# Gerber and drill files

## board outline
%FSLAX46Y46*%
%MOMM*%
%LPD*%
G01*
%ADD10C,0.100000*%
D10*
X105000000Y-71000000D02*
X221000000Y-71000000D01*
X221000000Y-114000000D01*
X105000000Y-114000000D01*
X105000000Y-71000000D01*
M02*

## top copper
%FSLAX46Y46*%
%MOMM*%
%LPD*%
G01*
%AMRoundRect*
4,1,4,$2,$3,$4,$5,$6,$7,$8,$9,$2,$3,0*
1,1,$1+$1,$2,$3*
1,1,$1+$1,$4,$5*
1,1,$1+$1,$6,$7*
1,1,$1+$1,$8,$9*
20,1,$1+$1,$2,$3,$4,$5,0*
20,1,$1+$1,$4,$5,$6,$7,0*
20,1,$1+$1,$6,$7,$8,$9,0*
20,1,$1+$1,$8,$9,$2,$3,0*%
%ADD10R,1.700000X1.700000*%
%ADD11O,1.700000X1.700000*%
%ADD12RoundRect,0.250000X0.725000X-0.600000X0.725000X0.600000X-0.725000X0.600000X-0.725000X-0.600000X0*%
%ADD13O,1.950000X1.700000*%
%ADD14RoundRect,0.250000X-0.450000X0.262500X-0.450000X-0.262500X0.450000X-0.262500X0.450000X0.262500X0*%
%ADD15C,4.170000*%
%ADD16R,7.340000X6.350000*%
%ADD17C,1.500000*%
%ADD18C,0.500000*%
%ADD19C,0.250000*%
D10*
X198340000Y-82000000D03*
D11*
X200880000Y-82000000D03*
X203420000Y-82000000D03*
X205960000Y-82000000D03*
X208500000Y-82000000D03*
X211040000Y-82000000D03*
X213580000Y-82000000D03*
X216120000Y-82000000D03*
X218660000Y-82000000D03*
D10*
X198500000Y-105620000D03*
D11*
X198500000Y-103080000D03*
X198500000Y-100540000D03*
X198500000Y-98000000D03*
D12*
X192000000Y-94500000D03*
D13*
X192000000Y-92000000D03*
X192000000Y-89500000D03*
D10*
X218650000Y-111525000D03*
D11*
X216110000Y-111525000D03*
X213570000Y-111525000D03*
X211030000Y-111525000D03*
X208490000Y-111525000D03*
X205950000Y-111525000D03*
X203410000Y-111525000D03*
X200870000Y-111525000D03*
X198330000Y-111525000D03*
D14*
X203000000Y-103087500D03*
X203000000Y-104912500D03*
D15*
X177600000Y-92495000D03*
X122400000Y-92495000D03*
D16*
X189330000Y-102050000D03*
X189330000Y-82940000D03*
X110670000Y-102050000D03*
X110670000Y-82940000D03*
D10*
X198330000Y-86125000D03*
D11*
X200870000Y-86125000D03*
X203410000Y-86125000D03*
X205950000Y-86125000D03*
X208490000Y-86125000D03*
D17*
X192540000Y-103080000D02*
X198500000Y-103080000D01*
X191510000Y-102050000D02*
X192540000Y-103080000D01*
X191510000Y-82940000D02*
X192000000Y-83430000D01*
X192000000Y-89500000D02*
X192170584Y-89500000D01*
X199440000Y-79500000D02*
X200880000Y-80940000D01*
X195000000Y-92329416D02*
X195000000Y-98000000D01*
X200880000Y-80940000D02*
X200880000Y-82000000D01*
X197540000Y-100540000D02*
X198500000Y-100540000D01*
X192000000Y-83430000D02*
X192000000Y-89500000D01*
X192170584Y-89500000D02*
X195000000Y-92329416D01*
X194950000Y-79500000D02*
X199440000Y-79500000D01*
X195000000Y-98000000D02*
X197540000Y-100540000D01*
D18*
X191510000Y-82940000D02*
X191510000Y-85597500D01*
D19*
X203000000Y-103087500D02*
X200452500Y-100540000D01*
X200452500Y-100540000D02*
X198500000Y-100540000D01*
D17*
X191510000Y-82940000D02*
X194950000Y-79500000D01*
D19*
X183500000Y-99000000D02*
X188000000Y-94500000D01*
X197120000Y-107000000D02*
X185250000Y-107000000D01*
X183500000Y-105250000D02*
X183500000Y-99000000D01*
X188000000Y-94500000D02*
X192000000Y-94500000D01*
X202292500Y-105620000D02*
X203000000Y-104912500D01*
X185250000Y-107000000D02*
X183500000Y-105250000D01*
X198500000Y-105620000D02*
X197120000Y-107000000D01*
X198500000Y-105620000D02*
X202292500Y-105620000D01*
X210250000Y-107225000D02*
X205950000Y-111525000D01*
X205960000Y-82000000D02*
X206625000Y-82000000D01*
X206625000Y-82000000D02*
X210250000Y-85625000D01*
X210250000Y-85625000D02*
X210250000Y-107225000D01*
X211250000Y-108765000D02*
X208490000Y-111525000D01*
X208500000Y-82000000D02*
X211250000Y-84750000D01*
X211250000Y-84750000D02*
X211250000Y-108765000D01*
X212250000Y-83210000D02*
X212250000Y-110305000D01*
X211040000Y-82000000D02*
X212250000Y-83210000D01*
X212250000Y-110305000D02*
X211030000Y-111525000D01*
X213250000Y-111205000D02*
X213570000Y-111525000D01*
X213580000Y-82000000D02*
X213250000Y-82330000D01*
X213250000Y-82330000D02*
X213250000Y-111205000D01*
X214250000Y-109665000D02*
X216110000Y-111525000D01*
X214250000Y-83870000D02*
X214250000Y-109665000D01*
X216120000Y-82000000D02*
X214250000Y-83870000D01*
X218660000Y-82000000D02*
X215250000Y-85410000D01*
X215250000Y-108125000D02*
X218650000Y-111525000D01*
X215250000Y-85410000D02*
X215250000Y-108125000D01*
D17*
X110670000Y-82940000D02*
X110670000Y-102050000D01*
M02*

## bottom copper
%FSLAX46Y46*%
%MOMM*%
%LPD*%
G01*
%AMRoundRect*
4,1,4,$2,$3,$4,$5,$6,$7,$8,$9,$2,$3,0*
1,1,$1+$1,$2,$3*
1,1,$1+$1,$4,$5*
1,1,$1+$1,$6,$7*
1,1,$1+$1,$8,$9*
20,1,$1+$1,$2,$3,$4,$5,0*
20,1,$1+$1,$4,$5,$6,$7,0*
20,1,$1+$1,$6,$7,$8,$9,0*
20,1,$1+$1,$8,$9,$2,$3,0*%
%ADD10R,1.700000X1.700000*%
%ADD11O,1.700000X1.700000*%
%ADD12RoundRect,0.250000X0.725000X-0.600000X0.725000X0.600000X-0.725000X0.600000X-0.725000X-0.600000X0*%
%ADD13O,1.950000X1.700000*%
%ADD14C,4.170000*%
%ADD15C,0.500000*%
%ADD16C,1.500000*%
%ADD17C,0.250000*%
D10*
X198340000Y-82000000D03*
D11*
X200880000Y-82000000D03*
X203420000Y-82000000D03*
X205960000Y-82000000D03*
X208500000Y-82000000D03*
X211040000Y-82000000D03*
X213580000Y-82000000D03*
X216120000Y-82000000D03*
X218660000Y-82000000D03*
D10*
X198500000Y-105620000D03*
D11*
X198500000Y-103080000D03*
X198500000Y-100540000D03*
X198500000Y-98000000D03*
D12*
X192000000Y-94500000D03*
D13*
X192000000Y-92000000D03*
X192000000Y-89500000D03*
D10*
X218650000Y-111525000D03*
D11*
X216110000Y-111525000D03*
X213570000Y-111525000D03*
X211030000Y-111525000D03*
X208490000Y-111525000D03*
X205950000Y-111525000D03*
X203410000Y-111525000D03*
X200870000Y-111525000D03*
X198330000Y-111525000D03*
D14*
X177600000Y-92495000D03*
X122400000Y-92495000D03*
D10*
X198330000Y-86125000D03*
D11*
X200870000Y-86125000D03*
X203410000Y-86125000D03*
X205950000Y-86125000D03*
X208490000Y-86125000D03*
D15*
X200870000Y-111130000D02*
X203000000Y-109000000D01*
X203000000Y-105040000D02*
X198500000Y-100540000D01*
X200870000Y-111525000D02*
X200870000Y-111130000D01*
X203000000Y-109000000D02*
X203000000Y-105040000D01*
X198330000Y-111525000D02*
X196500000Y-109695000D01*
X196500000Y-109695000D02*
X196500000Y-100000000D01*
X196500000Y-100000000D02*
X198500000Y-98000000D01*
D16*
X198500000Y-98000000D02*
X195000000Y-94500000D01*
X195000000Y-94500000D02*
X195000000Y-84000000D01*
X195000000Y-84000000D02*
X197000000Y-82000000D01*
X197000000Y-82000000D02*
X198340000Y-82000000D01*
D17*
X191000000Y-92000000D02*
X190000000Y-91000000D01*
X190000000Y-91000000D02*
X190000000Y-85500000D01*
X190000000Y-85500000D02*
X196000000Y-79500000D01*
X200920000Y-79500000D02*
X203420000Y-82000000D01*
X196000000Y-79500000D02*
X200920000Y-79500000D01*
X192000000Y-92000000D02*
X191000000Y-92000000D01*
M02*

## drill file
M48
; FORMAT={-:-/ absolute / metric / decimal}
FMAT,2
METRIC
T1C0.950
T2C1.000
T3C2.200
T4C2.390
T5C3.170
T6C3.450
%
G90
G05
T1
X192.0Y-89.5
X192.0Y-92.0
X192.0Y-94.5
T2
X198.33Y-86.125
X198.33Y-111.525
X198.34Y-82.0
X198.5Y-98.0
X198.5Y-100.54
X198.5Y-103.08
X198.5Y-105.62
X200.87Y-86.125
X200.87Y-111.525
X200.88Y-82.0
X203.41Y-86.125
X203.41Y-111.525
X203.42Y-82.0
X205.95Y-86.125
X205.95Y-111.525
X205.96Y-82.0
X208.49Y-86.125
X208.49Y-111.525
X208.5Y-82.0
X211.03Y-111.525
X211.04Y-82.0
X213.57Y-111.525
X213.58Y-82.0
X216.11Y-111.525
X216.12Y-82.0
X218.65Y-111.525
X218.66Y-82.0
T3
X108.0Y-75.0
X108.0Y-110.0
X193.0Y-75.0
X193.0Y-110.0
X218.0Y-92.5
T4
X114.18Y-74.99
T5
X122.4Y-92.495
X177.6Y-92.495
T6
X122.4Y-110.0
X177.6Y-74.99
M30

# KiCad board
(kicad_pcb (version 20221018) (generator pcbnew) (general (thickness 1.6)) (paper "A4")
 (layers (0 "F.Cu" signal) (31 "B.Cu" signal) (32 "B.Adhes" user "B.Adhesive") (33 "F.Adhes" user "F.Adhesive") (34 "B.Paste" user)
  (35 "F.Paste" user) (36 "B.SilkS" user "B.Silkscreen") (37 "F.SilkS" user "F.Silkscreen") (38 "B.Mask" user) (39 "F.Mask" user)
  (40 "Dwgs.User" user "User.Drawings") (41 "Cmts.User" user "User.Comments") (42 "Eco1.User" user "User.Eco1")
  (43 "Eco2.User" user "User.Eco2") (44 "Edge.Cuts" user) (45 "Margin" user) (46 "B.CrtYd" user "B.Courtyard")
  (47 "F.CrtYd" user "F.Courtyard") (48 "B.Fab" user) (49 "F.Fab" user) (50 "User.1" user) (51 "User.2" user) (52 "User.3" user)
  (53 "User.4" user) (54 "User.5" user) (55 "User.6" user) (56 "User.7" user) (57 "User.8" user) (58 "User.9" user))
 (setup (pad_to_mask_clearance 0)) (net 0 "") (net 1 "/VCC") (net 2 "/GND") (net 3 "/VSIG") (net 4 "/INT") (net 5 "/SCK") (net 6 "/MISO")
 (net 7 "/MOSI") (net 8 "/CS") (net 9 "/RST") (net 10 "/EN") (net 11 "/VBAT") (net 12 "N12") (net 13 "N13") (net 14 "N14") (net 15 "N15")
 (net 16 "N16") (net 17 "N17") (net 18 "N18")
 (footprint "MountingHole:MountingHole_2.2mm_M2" (layer "F.Cu") (at 108 110)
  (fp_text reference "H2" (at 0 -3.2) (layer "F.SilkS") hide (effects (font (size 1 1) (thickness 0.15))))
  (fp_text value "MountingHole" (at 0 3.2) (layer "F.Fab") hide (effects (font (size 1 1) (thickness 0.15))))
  (pad "" np_thru_hole circle (at 0 0) (size 2.2 2.2) (drill 2.2) (layers "*.Cu" "*.Mask")))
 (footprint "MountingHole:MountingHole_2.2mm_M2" (layer "F.Cu") (at 218 92.5)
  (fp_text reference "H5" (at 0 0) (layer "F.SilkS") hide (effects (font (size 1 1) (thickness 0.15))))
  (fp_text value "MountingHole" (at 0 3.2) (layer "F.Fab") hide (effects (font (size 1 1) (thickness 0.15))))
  (pad "" np_thru_hole circle (at 0 0) (size 2.2 2.2) (drill 2.2) (layers "*.Cu" "*.Mask")))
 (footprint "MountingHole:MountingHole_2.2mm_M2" (layer "F.Cu") (at 108 75)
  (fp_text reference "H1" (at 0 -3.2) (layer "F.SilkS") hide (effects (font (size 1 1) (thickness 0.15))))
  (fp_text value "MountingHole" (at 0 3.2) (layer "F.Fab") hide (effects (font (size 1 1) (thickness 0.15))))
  (pad "" np_thru_hole circle (at 0 0) (size 2.2 2.2) (drill 2.2) (layers "*.Cu" "*.Mask")))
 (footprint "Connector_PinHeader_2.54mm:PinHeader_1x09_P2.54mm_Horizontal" (layer "F.Cu") (at 198.34 82 90)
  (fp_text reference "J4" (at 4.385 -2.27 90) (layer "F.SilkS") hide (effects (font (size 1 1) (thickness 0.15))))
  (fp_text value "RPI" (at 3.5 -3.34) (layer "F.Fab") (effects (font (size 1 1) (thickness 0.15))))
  (pad "1" thru_hole rect (at 0 0 90) (size 1.7 1.7) (drill 1) (layers "*.Cu" "*.Mask") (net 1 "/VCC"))
  (pad "2" thru_hole oval (at 0 2.54 90) (size 1.7 1.7) (drill 1) (layers "*.Cu" "*.Mask") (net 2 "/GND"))
  (pad "3" thru_hole oval (at 0 5.08 90) (size 1.7 1.7) (drill 1) (layers "*.Cu" "*.Mask") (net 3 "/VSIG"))
  (pad "4" thru_hole oval (at 0 7.62 90) (size 1.7 1.7) (drill 1) (layers "*.Cu" "*.Mask") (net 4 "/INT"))
  (pad "5" thru_hole oval (at 0 10.16 90) (size 1.7 1.7) (drill 1) (layers "*.Cu" "*.Mask") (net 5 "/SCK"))
  (pad "6" thru_hole oval (at 0 12.7 90) (size 1.7 1.7) (drill 1) (layers "*.Cu" "*.Mask") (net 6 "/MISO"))
  (pad "7" thru_hole oval (at 0 15.24 90) (size 1.7 1.7) (drill 1) (layers "*.Cu" "*.Mask") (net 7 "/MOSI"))
  (pad "8" thru_hole oval (at 0 17.78 90) (size 1.7 1.7) (drill 1) (layers "*.Cu" "*.Mask") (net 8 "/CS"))
  (pad "9" thru_hole oval (at 0 20.32 90) (size 1.7 1.7) (drill 1) (layers "*.Cu" "*.Mask") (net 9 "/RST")))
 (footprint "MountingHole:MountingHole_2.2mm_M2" (layer "F.Cu") (at 193 110)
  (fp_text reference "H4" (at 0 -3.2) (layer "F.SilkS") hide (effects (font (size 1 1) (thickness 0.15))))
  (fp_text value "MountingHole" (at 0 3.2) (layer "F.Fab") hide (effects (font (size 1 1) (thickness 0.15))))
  (pad "" np_thru_hole circle (at 0 0) (size 2.2 2.2) (drill 2.2) (layers "*.Cu" "*.Mask")))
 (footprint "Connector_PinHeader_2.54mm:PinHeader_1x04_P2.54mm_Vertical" (layer "F.Cu") (at 198.5 105.62 180)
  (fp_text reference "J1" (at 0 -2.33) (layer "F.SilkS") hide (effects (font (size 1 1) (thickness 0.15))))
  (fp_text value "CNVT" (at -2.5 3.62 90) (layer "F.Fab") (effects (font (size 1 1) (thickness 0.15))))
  (pad "1" thru_hole rect (at 0 0 180) (size 1.7 1.7) (drill 1) (layers "*.Cu" "*.Mask") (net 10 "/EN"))
  (pad "2" thru_hole oval (at 0 2.54 180) (size 1.7 1.7) (drill 1) (layers "*.Cu" "*.Mask") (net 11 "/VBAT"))
  (pad "3" thru_hole oval (at 0 5.08 180) (size 1.7 1.7) (drill 1) (layers "*.Cu" "*.Mask") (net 2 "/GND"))
  (pad "4" thru_hole oval (at 0 7.62 180) (size 1.7 1.7) (drill 1) (layers "*.Cu" "*.Mask") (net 1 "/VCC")))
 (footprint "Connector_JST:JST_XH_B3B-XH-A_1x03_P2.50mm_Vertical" (layer "F.Cu") (at 192 94.5 90)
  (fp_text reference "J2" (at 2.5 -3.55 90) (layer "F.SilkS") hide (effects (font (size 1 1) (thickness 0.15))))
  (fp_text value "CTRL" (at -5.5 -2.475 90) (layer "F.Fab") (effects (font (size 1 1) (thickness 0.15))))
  (pad "1" thru_hole roundrect (at 0 0 90) (size 1.7 1.95) (drill 0.95) (layers "*.Cu" "*.Mask") (roundrect_rratio 0.147059) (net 10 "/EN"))
  (pad "2" thru_hole oval (at 2.5 0 90) (size 1.7 1.95) (drill 0.95) (layers "*.Cu" "*.Mask") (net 3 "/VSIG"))
  (pad "3" thru_hole oval (at 5 0 90) (size 1.7 1.95) (drill 0.95) (layers "*.Cu" "*.Mask") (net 2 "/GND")))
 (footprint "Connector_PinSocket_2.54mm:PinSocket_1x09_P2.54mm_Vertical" (layer "F.Cu") (at 218.65 111.525 -90)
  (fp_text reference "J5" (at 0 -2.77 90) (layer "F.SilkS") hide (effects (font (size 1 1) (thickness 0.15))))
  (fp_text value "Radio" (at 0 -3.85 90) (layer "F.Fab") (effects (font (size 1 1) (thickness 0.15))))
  (pad "1" thru_hole rect (at 0 0 270) (size 1.7 1.7) (drill 1) (layers "*.Cu" "*.Mask") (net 9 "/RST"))
  (pad "2" thru_hole oval (at 0 2.54 270) (size 1.7 1.7) (drill 1) (layers "*.Cu" "*.Mask") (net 8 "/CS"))
  (pad "3" thru_hole oval (at 0 5.08 270) (size 1.7 1.7) (drill 1) (layers "*.Cu" "*.Mask") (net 7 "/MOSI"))
  (pad "4" thru_hole oval (at 0 7.62 270) (size 1.7 1.7) (drill 1) (layers "*.Cu" "*.Mask") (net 6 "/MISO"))
  (pad "5" thru_hole oval (at 0 10.16 270) (size 1.7 1.7) (drill 1) (layers "*.Cu" "*.Mask") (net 5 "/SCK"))
  (pad "6" thru_hole oval (at 0 12.7 270) (size 1.7 1.7) (drill 1) (layers "*.Cu" "*.Mask") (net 4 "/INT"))
  (pad "7" thru_hole oval (at 0 15.24 270) (size 1.7 1.7) (drill 1) (layers "*.Cu" "*.Mask") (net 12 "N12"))
  (pad "8" thru_hole oval (at 0 17.78 270) (size 1.7 1.7) (drill 1) (layers "*.Cu" "*.Mask") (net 2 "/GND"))
  (pad "9" thru_hole oval (at 0 20.32 270) (size 1.7 1.7) (drill 1) (layers "*.Cu" "*.Mask") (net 1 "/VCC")))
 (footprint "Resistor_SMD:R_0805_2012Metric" (layer "F.Cu") (at 203 104 -90)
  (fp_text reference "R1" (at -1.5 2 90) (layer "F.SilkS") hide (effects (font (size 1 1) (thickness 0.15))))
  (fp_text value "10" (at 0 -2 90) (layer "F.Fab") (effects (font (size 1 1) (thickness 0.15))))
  (pad "1" smd roundrect (at -0.9125 0 270) (size 1.025 1.4) (layers "F.Cu" "F.Paste" "F.Mask") (roundrect_rratio 0.243902) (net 2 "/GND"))
  (pad "2" smd roundrect (at 0.9125 0 270) (size 1.025 1.4) (layers "F.Cu" "F.Paste" "F.Mask") (roundrect_rratio 0.243902) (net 10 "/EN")))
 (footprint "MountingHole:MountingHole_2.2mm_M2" (layer "F.Cu") (at 193 75)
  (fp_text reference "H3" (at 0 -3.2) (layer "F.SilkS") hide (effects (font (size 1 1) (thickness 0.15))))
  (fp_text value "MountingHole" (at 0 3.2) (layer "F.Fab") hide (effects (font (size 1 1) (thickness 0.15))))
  (pad "" np_thru_hole circle (at 0 0) (size 2.2 2.2) (drill 2.2) (layers "*.Cu" "*.Mask")))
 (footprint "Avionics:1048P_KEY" (layer "F.Cu") (at 150 92.495 180)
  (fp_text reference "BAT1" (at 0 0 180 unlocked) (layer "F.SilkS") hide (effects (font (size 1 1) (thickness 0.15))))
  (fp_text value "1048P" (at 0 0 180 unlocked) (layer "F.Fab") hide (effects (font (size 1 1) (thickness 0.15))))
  (pad "" np_thru_hole circle (at -27.6 0 180) (size 4.17 4.17) (drill 3.17) (layers "F&B.Cu" "*.Mask"))
  (pad "" np_thru_hole circle (at -27.6 17.505 180) (size 3.45 3.45) (drill 3.45) (layers "F&B.Cu" "*.Mask"))
  (pad "" np_thru_hole circle (at 27.6 -17.505 180) (size 3.45 3.45) (drill 3.45) (layers "F&B.Cu" "*.Mask"))
  (pad "" np_thru_hole circle (at 27.6 0 180) (size 4.17 4.17) (drill 3.17) (layers "F&B.Cu" "*.Mask"))
  (pad "" np_thru_hole circle (at 35.82 17.505 180) (size 2.39 2.39) (drill 2.39) (layers "F&B.Cu" "*.Mask"))
  (pad "1" smd rect (at -39.33 -9.555 180) (size 7.34 6.35) (layers "F.Cu" "F.Paste" "F.Mask") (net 11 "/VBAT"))
  (pad "2" smd rect (at -39.33 9.555 180) (size 7.34 6.35) (layers "F.Cu" "F.Paste" "F.Mask") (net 2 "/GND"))
  (pad "3" smd rect (at 39.33 -9.555 180) (size 7.34 6.35) (layers "F.Cu" "F.Paste" "F.Mask") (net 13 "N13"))
  (pad "4" smd rect (at 39.33 9.555 180) (size 7.34 6.35) (layers "F.Cu" "F.Paste" "F.Mask") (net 13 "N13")))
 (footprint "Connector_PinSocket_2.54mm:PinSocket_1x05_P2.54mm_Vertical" (layer "F.Cu") (at 198.33 86.125 90)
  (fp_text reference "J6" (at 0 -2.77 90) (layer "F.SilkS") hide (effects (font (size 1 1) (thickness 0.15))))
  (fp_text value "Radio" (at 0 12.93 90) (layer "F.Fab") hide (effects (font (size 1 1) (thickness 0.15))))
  (pad "1" thru_hole rect (at 0 0 90) (size 1.7 1.7) (drill 1) (layers "*.Cu" "*.Mask") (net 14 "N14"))
  (pad "2" thru_hole oval (at 0 2.54 90) (size 1.7 1.7) (drill 1) (layers "*.Cu" "*.Mask") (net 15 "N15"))
  (pad "3" thru_hole oval (at 0 5.08 90) (size 1.7 1.7) (drill 1) (layers "*.Cu" "*.Mask") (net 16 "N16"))
  (pad "4" thru_hole oval (at 0 7.62 90) (size 1.7 1.7) (drill 1) (layers "*.Cu" "*.Mask") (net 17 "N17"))
  (pad "5" thru_hole oval (at 0 10.16 90) (size 1.7 1.7) (drill 1) (layers "*.Cu" "*.Mask") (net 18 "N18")))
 (gr_rect (start 105 71) (end 221 114) (stroke (width 0.1) (type default)) (fill none) (layer "Edge.Cuts"))
 (segment (start 192.54 103.08) (end 198.5 103.08) (width 1.5) (layer "F.Cu") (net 11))
 (segment (start 191.51 102.05) (end 192.54 103.08) (width 1.5) (layer "F.Cu") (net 11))
 (segment (start 191.51 82.94) (end 192 83.43) (width 1.5) (layer "F.Cu") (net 2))
 (segment (start 192 89.5) (end 192.170584 89.5) (width 1.5) (layer "F.Cu") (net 2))
 (segment (start 199.44 79.5) (end 200.88 80.94) (width 1.5) (layer "F.Cu") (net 2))
 (segment (start 195 92.329416) (end 195 98) (width 1.5) (layer "F.Cu") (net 2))
 (segment (start 200.88 80.94) (end 200.88 82) (width 1.5) (layer "F.Cu") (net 2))
 (segment (start 197.54 100.54) (end 198.5 100.54) (width 1.5) (layer "F.Cu") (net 2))
 (segment (start 192 83.43) (end 192 89.5) (width 1.5) (layer "F.Cu") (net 2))
 (segment (start 192.170584 89.5) (end 195 92.329416) (width 1.5) (layer "F.Cu") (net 2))
 (segment (start 194.95 79.5) (end 199.44 79.5) (width 1.5) (layer "F.Cu") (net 2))
 (segment (start 195 98) (end 197.54 100.54) (width 1.5) (layer "F.Cu") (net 2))
 (segment (start 191.51 82.94) (end 191.51 85.5975) (width 0.5) (layer "F.Cu") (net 2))
 (segment (start 203 103.0875) (end 200.4525 100.54) (width 0.25) (layer "F.Cu") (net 2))
 (segment (start 200.4525 100.54) (end 198.5 100.54) (width 0.25) (layer "F.Cu") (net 2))
 (segment (start 191.51 82.94) (end 194.95 79.5) (width 1.5) (layer "F.Cu") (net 2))
 (segment (start 200.87 111.13) (end 203 109) (width 0.5) (layer "B.Cu") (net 2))
 (segment (start 203 105.04) (end 198.5 100.54) (width 0.5) (layer "B.Cu") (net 2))
 (segment (start 200.87 111.525) (end 200.87 111.13) (width 0.5) (layer "B.Cu") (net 2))
 (segment (start 203 109) (end 203 105.04) (width 0.5) (layer "B.Cu") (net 2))
 (segment (start 183.5 99) (end 188 94.5) (width 0.25) (layer "F.Cu") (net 10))
 (segment (start 197.12 107) (end 185.25 107) (width 0.25) (layer "F.Cu") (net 10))
 (segment (start 183.5 105.25) (end 183.5 99) (width 0.25) (layer "F.Cu") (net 10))
 (segment (start 188 94.5) (end 192 94.5) (width 0.25) (layer "F.Cu") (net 10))
 (segment (start 202.2925 105.62) (end 203 104.9125) (width 0.25) (layer "F.Cu") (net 10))
 (segment (start 185.25 107) (end 183.5 105.25) (width 0.25) (layer "F.Cu") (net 10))
 (segment (start 198.5 105.62) (end 197.12 107) (width 0.25) (layer "F.Cu") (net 10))
 (segment (start 198.5 105.62) (end 202.2925 105.62) (width 0.25) (layer "F.Cu") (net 10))
 (segment (start 198.33 111.525) (end 196.5 109.695) (width 0.5) (layer "B.Cu") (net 1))
 (segment (start 196.5 109.695) (end 196.5 100) (width 0.5) (layer "B.Cu") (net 1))
 (segment (start 196.5 100) (end 198.5 98) (width 0.5) (layer "B.Cu") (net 1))
 (segment (start 198.5 98) (end 195 94.5) (width 1.5) (layer "B.Cu") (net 1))
 (segment (start 195 94.5) (end 195 84) (width 1.5) (layer "B.Cu") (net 1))
 (segment (start 195 84) (end 197 82) (width 1.5) (layer "B.Cu") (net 1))
 (segment (start 197 82) (end 198.34 82) (width 1.5) (layer "B.Cu") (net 1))
 (segment (start 191 92) (end 190 91) (width 0.25) (layer "B.Cu") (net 3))
 (segment (start 190 91) (end 190 85.5) (width 0.25) (layer "B.Cu") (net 3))
 (segment (start 190 85.5) (end 196 79.5) (width 0.25) (layer "B.Cu") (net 3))
 (segment (start 200.92 79.5) (end 203.42 82) (width 0.25) (layer "B.Cu") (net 3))
 (segment (start 196 79.5) (end 200.92 79.5) (width 0.25) (layer "B.Cu") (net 3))
 (segment (start 192 92) (end 191 92) (width 0.25) (layer "B.Cu") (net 3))
 (segment (start 210.25 107.225) (end 205.95 111.525) (width 0.25) (layer "F.Cu") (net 4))
 (segment (start 205.96 82) (end 206.625 82) (width 0.25) (layer "F.Cu") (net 4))
 (segment (start 206.625 82) (end 210.25 85.625) (width 0.25) (layer "F.Cu") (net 4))
 (segment (start 210.25 85.625) (end 210.25 107.225) (width 0.25) (layer "F.Cu") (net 4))
 (segment (start 211.25 108.765) (end 208.49 111.525) (width 0.25) (layer "F.Cu") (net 5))
 (segment (start 208.5 82) (end 211.25 84.75) (width 0.25) (layer "F.Cu") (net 5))
 (segment (start 211.25 84.75) (end 211.25 108.765) (width 0.25) (layer "F.Cu") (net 5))
 (segment (start 212.25 83.21) (end 212.25 110.305) (width 0.25) (layer "F.Cu") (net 6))
 (segment (start 211.04 82) (end 212.25 83.21) (width 0.25) (layer "F.Cu") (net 6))
 (segment (start 212.25 110.305) (end 211.03 111.525) (width 0.25) (layer "F.Cu") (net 6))
 (segment (start 213.25 111.205) (end 213.57 111.525) (width 0.25) (layer "F.Cu") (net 7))
 (segment (start 213.58 82) (end 213.25 82.33) (width 0.25) (layer "F.Cu") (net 7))
 (segment (start 213.25 82.33) (end 213.25 111.205) (width 0.25) (layer "F.Cu") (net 7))
 (segment (start 214.25 109.665) (end 216.11 111.525) (width 0.25) (layer "F.Cu") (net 8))
 (segment (start 214.25 83.87) (end 214.25 109.665) (width 0.25) (layer "F.Cu") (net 8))
 (segment (start 216.12 82) (end 214.25 83.87) (width 0.25) (layer "F.Cu") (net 8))
 (segment (start 218.66 82) (end 215.25 85.41) (width 0.25) (layer "F.Cu") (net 9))
 (segment (start 215.25 108.125) (end 218.65 111.525) (width 0.25) (layer "F.Cu") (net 9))
 (segment (start 215.25 85.41) (end 215.25 108.125) (width 0.25) (layer "F.Cu") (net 9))
 (segment (start 110.67 82.94) (end 110.67 102.05) (width 1.5) (layer "F.Cu") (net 13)))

